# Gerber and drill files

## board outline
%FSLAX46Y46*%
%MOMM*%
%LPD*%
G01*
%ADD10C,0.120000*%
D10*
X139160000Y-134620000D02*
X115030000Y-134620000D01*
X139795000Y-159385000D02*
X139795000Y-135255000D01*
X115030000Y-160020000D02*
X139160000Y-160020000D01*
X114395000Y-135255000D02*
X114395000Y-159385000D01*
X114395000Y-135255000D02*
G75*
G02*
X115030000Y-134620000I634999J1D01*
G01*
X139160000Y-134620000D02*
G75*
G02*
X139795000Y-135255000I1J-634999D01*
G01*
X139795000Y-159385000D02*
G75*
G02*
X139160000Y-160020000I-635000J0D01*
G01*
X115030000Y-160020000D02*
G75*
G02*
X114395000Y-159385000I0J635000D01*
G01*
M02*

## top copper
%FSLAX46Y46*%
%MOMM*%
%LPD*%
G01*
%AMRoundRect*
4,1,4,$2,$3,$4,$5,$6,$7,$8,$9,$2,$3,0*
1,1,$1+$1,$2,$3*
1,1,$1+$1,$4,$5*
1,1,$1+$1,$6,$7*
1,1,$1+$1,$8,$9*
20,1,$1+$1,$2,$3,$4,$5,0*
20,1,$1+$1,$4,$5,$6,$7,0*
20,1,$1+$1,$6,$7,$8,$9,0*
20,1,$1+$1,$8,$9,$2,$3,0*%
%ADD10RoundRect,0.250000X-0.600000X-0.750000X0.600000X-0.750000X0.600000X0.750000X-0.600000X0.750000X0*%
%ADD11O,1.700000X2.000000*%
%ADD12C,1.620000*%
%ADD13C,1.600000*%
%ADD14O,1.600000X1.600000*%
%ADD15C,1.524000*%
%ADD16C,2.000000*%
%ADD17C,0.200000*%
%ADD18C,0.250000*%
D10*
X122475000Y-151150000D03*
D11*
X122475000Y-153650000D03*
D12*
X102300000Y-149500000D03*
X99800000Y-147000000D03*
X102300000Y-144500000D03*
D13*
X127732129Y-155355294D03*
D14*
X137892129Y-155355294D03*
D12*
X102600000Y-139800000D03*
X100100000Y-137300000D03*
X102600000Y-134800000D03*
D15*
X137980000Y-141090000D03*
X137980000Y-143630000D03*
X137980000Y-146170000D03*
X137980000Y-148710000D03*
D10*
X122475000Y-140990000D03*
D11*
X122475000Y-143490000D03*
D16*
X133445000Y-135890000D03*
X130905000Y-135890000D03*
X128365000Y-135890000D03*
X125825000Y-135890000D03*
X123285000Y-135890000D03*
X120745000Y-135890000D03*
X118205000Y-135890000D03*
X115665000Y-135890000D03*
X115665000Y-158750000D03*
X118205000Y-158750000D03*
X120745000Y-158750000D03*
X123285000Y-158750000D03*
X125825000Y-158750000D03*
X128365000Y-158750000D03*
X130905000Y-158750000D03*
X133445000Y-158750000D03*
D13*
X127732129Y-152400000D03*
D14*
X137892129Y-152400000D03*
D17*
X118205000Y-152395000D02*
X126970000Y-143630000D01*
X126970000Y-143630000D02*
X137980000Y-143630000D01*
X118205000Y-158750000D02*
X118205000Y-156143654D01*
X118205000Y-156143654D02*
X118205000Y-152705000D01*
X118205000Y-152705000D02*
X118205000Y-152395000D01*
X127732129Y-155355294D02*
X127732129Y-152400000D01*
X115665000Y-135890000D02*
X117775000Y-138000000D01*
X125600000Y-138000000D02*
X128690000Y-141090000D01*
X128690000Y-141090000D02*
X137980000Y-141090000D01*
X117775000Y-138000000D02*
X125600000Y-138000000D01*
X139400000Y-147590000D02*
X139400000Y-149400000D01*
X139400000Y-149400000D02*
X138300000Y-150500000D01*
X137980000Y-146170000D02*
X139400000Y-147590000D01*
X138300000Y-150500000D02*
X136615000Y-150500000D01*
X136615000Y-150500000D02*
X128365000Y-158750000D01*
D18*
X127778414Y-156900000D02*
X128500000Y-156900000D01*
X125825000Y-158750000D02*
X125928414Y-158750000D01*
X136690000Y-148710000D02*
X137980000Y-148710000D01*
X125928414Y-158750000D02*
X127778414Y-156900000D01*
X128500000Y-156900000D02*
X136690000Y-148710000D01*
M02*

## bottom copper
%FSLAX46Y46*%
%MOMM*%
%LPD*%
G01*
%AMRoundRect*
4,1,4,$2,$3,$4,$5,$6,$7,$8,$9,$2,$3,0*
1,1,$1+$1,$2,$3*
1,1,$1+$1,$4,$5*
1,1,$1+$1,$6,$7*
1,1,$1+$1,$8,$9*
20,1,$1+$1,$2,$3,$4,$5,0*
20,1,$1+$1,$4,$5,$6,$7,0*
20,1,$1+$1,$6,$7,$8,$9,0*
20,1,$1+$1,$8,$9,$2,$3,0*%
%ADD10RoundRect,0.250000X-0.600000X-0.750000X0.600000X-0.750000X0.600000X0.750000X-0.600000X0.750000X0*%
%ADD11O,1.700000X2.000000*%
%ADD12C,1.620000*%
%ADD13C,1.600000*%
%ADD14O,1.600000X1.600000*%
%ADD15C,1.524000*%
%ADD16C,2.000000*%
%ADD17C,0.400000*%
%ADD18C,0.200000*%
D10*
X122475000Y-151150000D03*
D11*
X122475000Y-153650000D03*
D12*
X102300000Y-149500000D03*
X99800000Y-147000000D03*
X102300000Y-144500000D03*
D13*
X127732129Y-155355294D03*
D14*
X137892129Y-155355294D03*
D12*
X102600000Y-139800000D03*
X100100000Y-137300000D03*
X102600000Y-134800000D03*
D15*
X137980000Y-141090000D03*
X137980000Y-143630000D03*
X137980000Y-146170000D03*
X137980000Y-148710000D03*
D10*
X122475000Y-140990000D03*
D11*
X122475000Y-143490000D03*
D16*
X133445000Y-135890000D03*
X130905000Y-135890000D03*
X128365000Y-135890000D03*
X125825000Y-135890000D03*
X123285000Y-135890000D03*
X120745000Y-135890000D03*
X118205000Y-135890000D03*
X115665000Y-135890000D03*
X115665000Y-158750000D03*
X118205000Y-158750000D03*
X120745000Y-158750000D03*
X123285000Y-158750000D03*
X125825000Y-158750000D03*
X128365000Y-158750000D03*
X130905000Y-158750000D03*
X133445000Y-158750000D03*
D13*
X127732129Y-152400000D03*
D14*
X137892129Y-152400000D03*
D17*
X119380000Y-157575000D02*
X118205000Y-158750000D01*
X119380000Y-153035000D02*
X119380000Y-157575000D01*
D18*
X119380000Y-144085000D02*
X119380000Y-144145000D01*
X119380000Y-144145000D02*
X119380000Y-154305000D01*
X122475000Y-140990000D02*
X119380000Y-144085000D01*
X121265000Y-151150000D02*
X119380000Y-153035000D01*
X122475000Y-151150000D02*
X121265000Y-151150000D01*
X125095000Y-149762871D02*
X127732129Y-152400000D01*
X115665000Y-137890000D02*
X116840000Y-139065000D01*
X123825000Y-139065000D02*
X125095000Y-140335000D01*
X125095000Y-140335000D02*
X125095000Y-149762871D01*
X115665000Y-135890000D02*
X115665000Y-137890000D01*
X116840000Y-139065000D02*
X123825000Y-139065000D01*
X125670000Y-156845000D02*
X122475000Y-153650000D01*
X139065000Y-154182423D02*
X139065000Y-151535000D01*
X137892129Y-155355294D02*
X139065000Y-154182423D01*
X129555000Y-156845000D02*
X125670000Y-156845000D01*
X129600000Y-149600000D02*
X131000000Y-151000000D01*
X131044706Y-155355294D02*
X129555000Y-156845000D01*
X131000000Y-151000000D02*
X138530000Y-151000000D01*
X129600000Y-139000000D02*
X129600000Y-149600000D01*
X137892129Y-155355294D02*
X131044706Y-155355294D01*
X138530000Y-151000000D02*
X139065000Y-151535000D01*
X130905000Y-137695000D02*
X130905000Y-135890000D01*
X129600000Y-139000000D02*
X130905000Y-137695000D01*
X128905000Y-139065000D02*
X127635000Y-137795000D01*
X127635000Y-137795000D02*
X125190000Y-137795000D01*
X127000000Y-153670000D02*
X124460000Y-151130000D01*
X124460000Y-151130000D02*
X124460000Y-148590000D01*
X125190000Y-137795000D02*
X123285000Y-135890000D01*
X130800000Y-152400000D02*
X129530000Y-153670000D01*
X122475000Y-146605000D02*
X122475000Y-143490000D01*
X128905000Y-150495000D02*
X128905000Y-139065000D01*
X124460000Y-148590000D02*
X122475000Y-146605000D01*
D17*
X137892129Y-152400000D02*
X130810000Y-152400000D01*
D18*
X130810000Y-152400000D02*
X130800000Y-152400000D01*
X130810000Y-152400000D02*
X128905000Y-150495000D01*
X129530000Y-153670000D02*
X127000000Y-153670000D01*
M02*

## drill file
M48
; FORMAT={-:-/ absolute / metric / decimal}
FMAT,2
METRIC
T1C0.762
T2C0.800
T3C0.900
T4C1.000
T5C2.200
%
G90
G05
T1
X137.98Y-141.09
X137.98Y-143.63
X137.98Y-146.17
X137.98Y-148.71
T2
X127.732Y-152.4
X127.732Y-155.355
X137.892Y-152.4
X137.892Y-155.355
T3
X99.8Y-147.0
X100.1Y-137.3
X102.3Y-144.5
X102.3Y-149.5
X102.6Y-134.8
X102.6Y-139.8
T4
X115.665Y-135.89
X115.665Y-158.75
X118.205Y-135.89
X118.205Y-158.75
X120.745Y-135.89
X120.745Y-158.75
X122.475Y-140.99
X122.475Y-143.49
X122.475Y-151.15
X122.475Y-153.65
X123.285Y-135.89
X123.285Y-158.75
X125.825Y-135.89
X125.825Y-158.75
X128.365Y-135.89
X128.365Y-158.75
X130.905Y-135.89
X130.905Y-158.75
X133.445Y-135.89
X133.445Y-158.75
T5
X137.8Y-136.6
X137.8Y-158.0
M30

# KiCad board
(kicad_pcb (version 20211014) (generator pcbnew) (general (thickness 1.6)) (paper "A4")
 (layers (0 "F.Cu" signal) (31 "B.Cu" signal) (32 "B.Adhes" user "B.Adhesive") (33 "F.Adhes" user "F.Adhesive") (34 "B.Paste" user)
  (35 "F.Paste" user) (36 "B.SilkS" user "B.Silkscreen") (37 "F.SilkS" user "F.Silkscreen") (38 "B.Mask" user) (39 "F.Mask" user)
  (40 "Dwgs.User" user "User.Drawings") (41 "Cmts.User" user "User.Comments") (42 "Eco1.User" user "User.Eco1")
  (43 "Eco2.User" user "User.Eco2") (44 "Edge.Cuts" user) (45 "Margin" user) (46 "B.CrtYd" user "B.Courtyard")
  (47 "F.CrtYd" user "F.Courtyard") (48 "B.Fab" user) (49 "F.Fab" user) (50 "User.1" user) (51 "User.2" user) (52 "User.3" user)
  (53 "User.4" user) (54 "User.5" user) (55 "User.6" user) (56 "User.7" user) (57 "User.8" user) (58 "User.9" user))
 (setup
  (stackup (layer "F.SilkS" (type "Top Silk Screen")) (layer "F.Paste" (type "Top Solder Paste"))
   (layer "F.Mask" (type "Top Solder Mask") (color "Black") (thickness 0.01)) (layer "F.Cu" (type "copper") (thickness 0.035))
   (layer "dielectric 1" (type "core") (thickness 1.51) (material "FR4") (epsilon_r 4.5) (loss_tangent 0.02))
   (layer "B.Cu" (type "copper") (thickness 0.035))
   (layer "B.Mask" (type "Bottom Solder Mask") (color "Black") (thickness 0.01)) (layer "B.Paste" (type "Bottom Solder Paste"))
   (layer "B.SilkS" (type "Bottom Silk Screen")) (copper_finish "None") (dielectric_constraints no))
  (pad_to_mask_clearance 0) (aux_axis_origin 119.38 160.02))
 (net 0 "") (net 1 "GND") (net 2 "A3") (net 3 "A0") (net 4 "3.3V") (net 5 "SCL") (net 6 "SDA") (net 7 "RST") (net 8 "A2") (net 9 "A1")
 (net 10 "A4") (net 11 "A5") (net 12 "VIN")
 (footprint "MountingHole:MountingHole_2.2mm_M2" (layer "F.Cu") (at 137.8 136.6)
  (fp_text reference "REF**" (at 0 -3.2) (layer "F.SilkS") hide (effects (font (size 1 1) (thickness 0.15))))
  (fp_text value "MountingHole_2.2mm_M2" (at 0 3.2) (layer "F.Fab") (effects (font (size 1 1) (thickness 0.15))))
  (pad "" np_thru_hole circle (at 0 0) (size 2.2 2.2) (drill 2.2) (layers *.Cu *.Mask)))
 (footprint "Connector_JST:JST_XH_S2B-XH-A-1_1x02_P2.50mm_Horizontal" (layer "F.Cu") (at 114.375 152.4 -90)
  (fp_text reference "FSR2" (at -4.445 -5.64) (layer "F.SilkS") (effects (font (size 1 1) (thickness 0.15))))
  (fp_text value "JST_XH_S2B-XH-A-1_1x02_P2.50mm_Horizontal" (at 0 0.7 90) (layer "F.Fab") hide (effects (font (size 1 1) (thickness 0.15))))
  (pad "1" thru_hole roundrect (at -1.25 -8.1) (size 1.7 2) (drill 1) (layers *.Cu *.Mask) (roundrect_rratio 0.1470588235) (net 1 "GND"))
  (pad "2" thru_hole oval (at 1.25 -8.1) (size 1.7 2) (drill 1) (layers *.Cu *.Mask) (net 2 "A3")))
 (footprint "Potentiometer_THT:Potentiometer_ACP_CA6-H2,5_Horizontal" (layer "F.Cu") (at 102.3 149.5 180)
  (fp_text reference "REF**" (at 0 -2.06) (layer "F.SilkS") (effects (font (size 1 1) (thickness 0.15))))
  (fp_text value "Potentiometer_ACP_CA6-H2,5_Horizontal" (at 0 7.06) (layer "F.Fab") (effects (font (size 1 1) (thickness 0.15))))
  (pad "1" thru_hole circle (at 0 0 180) (size 1.62 1.62) (drill 0.9) (layers F&B.Cu *.Mask))
  (pad "2" thru_hole circle (at 2.5 2.5 180) (size 1.62 1.62) (drill 0.9) (layers *.Cu *.Mask) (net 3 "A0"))
  (pad "3" thru_hole circle (at 0 5 180) (size 1.62 1.62) (drill 0.9) (layers *.Cu *.Mask) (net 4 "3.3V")))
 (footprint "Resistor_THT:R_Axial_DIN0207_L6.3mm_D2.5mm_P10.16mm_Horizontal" (layer "F.Cu") (at 127.732129 155.355294)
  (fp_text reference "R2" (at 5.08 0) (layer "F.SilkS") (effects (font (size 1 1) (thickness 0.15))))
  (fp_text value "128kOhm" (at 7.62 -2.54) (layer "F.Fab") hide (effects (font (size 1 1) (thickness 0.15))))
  (pad "1" thru_hole circle (at 0 0) (size 1.6 1.6) (drill 0.8) (layers *.Cu *.Mask) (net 4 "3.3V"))
  (pad "2" thru_hole oval (at 10.16 0) (size 1.6 1.6) (drill 0.8) (layers *.Cu *.Mask) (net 2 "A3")))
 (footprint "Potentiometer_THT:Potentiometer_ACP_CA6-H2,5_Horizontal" (layer "F.Cu") (at 102.6 139.8 180)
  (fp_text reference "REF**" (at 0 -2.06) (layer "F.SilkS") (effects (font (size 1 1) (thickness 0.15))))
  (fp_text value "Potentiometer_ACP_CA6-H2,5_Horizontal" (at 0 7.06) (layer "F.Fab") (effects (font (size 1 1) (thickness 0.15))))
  (pad "1" thru_hole circle (at 0 0 180) (size 1.62 1.62) (drill 0.9) (layers *.Cu *.Mask))
  (pad "2" thru_hole circle (at 2.5 2.5 180) (size 1.62 1.62) (drill 0.9) (layers *.Cu *.Mask) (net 2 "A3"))
  (pad "3" thru_hole circle (at 0 5 180) (size 1.62 1.62) (drill 0.9) (layers *.Cu *.Mask) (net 4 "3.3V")))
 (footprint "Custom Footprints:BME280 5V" (layer "F.Cu") (at 136.71 144.9 -90)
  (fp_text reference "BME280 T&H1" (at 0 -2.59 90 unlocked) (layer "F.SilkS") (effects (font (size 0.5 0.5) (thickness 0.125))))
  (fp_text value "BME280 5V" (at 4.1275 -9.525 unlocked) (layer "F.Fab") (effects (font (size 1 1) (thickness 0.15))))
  (pad "1" thru_hole circle (at -3.81 -1.27 180) (size 1.524 1.524) (drill 0.762) (layers *.Cu *.Mask) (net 4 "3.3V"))
  (pad "2" thru_hole circle (at -1.27 -1.27 180) (size 1.524 1.524) (drill 0.762) (layers *.Cu *.Mask) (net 1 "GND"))
  (pad "3" thru_hole circle (at 1.27 -1.27 180) (size 1.524 1.524) (drill 0.762) (layers *.Cu *.Mask) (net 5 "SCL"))
  (pad "4" thru_hole circle (at 3.81 -1.27 180) (size 1.524 1.524) (drill 0.762) (layers *.Cu *.Mask) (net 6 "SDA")))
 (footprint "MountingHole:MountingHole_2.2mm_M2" (layer "F.Cu") (at 137.8 158)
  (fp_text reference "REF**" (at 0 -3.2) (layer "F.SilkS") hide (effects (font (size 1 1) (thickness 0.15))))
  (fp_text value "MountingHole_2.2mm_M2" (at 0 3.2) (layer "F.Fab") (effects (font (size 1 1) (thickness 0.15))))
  (pad "" np_thru_hole circle (at 0 0) (size 2.2 2.2) (drill 2.2) (layers *.Cu *.Mask)))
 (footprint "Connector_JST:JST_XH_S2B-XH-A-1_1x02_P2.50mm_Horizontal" (layer "F.Cu") (at 114.375 142.24 -90)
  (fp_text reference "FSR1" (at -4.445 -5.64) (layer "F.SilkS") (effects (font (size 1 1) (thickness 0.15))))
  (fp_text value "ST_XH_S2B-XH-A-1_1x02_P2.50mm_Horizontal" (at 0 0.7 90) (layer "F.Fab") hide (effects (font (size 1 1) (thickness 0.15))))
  (pad "1" thru_hole roundrect (at -1.25 -8.1) (size 1.7 2) (drill 1) (layers *.Cu *.Mask) (roundrect_rratio 0.1470588235) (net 1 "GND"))
  (pad "2" thru_hole oval (at 1.25 -8.1) (size 1.7 2) (drill 1) (layers *.Cu *.Mask) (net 3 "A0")))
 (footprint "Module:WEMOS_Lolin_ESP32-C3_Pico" (layer "F.Cu") (at 114.395 147.32 -90)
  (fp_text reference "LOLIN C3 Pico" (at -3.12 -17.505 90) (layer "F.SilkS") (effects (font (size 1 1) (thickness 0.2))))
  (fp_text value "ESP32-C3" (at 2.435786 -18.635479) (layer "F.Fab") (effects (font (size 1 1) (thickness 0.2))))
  (fp_line (start -12.7 -24.765) (end -12.7 -0.635) (layer "Edge.Cuts") (width 0.12))
  (fp_line (start 12.065 -25.4) (end -12.065 -25.4) (layer "Edge.Cuts") (width 0.12))
  (fp_line (start 12.7 -0.635) (end 12.7 -24.765) (layer "Edge.Cuts") (width 0.12))
  (fp_line (start -12.065 0) (end 12.065 0) (layer "Edge.Cuts") (width 0.12))
  (fp_arc (start -12.065 0) (mid -12.514013 -0.185987) (end -12.7 -0.635) (layer "Edge.Cuts") (width 0.12))
  (fp_arc (start -12.7 -24.765) (mid -12.514013 -25.214013) (end -12.065 -25.4) (layer "Edge.Cuts") (width 0.12))
  (fp_arc (start 12.065 -25.4) (mid 12.514013 -25.214013) (end 12.7 -24.765) (layer "Edge.Cuts") (width 0.12))
  (fp_arc (start 12.7 -0.635) (mid 12.514013 -0.185987) (end 12.065 0) (layer "Edge.Cuts") (width 0.12))
  (pad "1" thru_hole circle (at -11.43 -19.05 270) (size 2 2) (drill 1) (layers *.Cu *.Mask) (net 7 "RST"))
  (pad "2" thru_hole circle (at -11.43 -16.51 270) (size 2 2) (drill 1) (layers *.Cu *.Mask) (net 2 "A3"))
  (pad "3" thru_hole circle (at -11.43 -13.97 270) (size 2 2) (drill 1) (layers *.Cu *.Mask) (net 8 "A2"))
  (pad "4" thru_hole circle (at -11.43 -11.43 270) (size 2 2) (drill 1) (layers *.Cu *.Mask) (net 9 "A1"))
  (pad "5" thru_hole circle (at -11.43 -8.89 270) (size 2 2) (drill 1) (layers *.Cu *.Mask) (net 3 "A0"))
  (pad "6" thru_hole circle (at -11.43 -6.35 270) (size 2 2) (drill 1) (layers *.Cu *.Mask) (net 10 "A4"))
  (pad "7" thru_hole circle (at -11.43 -3.81 270) (size 2 2) (drill 1) (layers *.Cu *.Mask) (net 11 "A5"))
  (pad "8" thru_hole circle (at -11.43 -1.27 270) (size 2 2) (drill 1) (layers *.Cu *.Mask) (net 4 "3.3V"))
  (pad "9" thru_hole circle (at 11.43 -1.27 270) (size 2 2) (drill 1) (layers *.Cu *.Mask) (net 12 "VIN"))
  (pad "10" thru_hole circle (at 11.43 -3.81 270) (size 2 2) (drill 1) (layers *.Cu *.Mask) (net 1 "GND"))
  (pad "11" thru_hole circle (at 11.43 -6.35 270) (size 2 2) (drill 1) (layers *.Cu *.Mask))
  (pad "12" thru_hole circle (at 11.43 -8.89 270) (size 2 2) (drill 1) (layers *.Cu *.Mask))
  (pad "13" thru_hole circle (at 11.43 -11.43 270) (size 2 2) (drill 1) (layers *.Cu *.Mask) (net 6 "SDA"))
  (pad "14" thru_hole circle (at 11.43 -13.97 270) (size 2 2) (drill 1) (layers *.Cu *.Mask) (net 5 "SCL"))
  (pad "15" thru_hole circle (at 11.43 -16.51 270) (size 2 2) (drill 1) (layers *.Cu *.Mask))
  (pad "16" thru_hole circle (at 11.43 -19.05 270) (size 2 2) (drill 1) (layers *.Cu *.Mask)))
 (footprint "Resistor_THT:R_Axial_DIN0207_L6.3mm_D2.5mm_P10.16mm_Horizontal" (layer "F.Cu") (at 127.732129 152.4)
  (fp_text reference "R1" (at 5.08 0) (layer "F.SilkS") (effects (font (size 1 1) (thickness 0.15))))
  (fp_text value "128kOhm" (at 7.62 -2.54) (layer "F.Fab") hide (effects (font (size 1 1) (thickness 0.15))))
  (pad "1" thru_hole circle (at 0 0) (size 1.6 1.6) (drill 0.8) (layers *.Cu *.Mask) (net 4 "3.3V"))
  (pad "2" thru_hole oval (at 10.16 0) (size 1.6 1.6) (drill 0.8) (layers *.Cu *.Mask) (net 3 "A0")))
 (segment (start 118.205 152.395) (end 126.97 143.63) (width 0.2) (layer "F.Cu") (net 1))
 (segment (start 126.97 143.63) (end 137.98 143.63) (width 0.2) (layer "F.Cu") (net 1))
 (segment (start 118.205 158.75) (end 118.205 156.143654) (width 0.2) (layer "F.Cu") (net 1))
 (segment (start 118.205 156.143654) (end 118.205 152.705) (width 0.2) (layer "F.Cu") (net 1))
 (segment (start 118.205 152.705) (end 118.205 152.395) (width 0.2) (layer "F.Cu") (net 1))
 (segment (start 119.38 157.575) (end 118.205 158.75) (width 0.4) (layer "B.Cu") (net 1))
 (segment (start 119.38 153.035) (end 119.38 157.575) (width 0.4) (layer "B.Cu") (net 1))
 (segment (start 119.38 144.085) (end 119.38 144.145) (width 0.2) (layer "B.Cu") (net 1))
 (segment (start 119.38 144.145) (end 119.38 154.305) (width 0.2) (layer "B.Cu") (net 1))
 (segment (start 122.475 140.99) (end 119.38 144.085) (width 0.2) (layer "B.Cu") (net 1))
 (segment (start 121.265 151.15) (end 119.38 153.035) (width 0.2) (layer "B.Cu") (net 1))
 (segment (start 122.475 151.15) (end 121.265 151.15) (width 0.2) (layer "B.Cu") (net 1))
 (segment (start 127.732129 155.355294) (end 127.732129 152.4) (width 0.2) (layer "F.Cu") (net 4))
 (segment (start 115.665 135.89) (end 117.775 138) (width 0.2) (layer "F.Cu") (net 4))
 (segment (start 125.6 138) (end 128.69 141.09) (width 0.2) (layer "F.Cu") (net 4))
 (segment (start 128.69 141.09) (end 137.98 141.09) (width 0.2) (layer "F.Cu") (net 4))
 (segment (start 117.775 138) (end 125.6 138) (width 0.2) (layer "F.Cu") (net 4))
 (segment (start 125.095 149.762871) (end 127.732129 152.4) (width 0.2) (layer "B.Cu") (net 4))
 (segment (start 115.665 137.89) (end 116.84 139.065) (width 0.2) (layer "B.Cu") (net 4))
 (segment (start 123.825 139.065) (end 125.095 140.335) (width 0.2) (layer "B.Cu") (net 4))
 (segment (start 125.095 140.335) (end 125.095 149.762871) (width 0.2) (layer "B.Cu") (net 4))
 (segment (start 115.665 135.89) (end 115.665 137.89) (width 0.2) (layer "B.Cu") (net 4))
 (segment (start 116.84 139.065) (end 123.825 139.065) (width 0.2) (layer "B.Cu") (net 4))
 (segment (start 125.67 156.845) (end 122.475 153.65) (width 0.2) (layer "B.Cu") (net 2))
 (segment (start 139.065 154.182423) (end 139.065 151.535) (width 0.2) (layer "B.Cu") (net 2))
 (segment (start 137.892129 155.355294) (end 139.065 154.182423) (width 0.2) (layer "B.Cu") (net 2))
 (segment (start 129.555 156.845) (end 125.67 156.845) (width 0.2) (layer "B.Cu") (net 2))
 (segment (start 129.6 149.6) (end 131 151) (width 0.2) (layer "B.Cu") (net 2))
 (segment (start 131.044706 155.355294) (end 129.555 156.845) (width 0.2) (layer "B.Cu") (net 2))
 (segment (start 131 151) (end 138.53 151) (width 0.2) (layer "B.Cu") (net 2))
 (segment (start 129.6 139) (end 129.6 149.6) (width 0.2) (layer "B.Cu") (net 2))
 (segment (start 137.892129 155.355294) (end 131.044706 155.355294) (width 0.2) (layer "B.Cu") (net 2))
 (segment (start 138.53 151) (end 139.065 151.535) (width 0.2) (layer "B.Cu") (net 2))
 (segment (start 130.905 137.695) (end 130.905 135.89) (width 0.2) (layer "B.Cu") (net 2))
 (segment (start 129.6 139) (end 130.905 137.695) (width 0.2) (layer "B.Cu") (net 2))
 (segment (start 128.905 139.065) (end 127.635 137.795) (width 0.2) (layer "B.Cu") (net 3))
 (segment (start 127.635 137.795) (end 125.19 137.795) (width 0.2) (layer "B.Cu") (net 3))
 (segment (start 127 153.67) (end 124.46 151.13) (width 0.2) (layer "B.Cu") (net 3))
 (segment (start 124.46 151.13) (end 124.46 148.59) (width 0.2) (layer "B.Cu") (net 3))
 (segment (start 125.19 137.795) (end 123.285 135.89) (width 0.2) (layer "B.Cu") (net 3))
 (segment (start 130.8 152.4) (end 129.53 153.67) (width 0.2) (layer "B.Cu") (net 3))
 (segment (start 122.475 146.605) (end 122.475 143.49) (width 0.2) (layer "B.Cu") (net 3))
 (segment (start 128.905 150.495) (end 128.905 139.065) (width 0.2) (layer "B.Cu") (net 3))
 (segment (start 124.46 148.59) (end 122.475 146.605) (width 0.2) (layer "B.Cu") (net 3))
 (segment (start 137.892129 152.4) (end 130.81 152.4) (width 0.4) (layer "B.Cu") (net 3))
 (segment (start 130.81 152.4) (end 130.8 152.4) (width 0.2) (layer "B.Cu") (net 3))
 (segment (start 130.81 152.4) (end 128.905 150.495) (width 0.2) (layer "B.Cu") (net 3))
 (segment (start 129.53 153.67) (end 127 153.67) (width 0.2) (layer "B.Cu") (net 3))
 (segment (start 139.4 147.59) (end 139.4 149.4) (width 0.2) (layer "F.Cu") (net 5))
 (segment (start 139.4 149.4) (end 138.3 150.5) (width 0.2) (layer "F.Cu") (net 5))
 (segment (start 137.98 146.17) (end 139.4 147.59) (width 0.2) (layer "F.Cu") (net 5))
 (segment (start 138.3 150.5) (end 136.615 150.5) (width 0.2) (layer "F.Cu") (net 5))
 (segment (start 136.615 150.5) (end 128.365 158.75) (width 0.2) (layer "F.Cu") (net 5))
 (segment (start 127.778414 156.9) (end 128.5 156.9) (width 0.25) (layer "F.Cu") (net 6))
 (segment (start 125.825 158.75) (end 125.928414 158.75) (width 0.25) (layer "F.Cu") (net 6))
 (segment (start 136.69 148.71) (end 137.98 148.71) (width 0.25) (layer "F.Cu") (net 6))
 (segment (start 125.928414 158.75) (end 127.778414 156.9) (width 0.25) (layer "F.Cu") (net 6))
 (segment (start 128.5 156.9) (end 136.69 148.71) (width 0.25) (layer "F.Cu") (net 6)))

